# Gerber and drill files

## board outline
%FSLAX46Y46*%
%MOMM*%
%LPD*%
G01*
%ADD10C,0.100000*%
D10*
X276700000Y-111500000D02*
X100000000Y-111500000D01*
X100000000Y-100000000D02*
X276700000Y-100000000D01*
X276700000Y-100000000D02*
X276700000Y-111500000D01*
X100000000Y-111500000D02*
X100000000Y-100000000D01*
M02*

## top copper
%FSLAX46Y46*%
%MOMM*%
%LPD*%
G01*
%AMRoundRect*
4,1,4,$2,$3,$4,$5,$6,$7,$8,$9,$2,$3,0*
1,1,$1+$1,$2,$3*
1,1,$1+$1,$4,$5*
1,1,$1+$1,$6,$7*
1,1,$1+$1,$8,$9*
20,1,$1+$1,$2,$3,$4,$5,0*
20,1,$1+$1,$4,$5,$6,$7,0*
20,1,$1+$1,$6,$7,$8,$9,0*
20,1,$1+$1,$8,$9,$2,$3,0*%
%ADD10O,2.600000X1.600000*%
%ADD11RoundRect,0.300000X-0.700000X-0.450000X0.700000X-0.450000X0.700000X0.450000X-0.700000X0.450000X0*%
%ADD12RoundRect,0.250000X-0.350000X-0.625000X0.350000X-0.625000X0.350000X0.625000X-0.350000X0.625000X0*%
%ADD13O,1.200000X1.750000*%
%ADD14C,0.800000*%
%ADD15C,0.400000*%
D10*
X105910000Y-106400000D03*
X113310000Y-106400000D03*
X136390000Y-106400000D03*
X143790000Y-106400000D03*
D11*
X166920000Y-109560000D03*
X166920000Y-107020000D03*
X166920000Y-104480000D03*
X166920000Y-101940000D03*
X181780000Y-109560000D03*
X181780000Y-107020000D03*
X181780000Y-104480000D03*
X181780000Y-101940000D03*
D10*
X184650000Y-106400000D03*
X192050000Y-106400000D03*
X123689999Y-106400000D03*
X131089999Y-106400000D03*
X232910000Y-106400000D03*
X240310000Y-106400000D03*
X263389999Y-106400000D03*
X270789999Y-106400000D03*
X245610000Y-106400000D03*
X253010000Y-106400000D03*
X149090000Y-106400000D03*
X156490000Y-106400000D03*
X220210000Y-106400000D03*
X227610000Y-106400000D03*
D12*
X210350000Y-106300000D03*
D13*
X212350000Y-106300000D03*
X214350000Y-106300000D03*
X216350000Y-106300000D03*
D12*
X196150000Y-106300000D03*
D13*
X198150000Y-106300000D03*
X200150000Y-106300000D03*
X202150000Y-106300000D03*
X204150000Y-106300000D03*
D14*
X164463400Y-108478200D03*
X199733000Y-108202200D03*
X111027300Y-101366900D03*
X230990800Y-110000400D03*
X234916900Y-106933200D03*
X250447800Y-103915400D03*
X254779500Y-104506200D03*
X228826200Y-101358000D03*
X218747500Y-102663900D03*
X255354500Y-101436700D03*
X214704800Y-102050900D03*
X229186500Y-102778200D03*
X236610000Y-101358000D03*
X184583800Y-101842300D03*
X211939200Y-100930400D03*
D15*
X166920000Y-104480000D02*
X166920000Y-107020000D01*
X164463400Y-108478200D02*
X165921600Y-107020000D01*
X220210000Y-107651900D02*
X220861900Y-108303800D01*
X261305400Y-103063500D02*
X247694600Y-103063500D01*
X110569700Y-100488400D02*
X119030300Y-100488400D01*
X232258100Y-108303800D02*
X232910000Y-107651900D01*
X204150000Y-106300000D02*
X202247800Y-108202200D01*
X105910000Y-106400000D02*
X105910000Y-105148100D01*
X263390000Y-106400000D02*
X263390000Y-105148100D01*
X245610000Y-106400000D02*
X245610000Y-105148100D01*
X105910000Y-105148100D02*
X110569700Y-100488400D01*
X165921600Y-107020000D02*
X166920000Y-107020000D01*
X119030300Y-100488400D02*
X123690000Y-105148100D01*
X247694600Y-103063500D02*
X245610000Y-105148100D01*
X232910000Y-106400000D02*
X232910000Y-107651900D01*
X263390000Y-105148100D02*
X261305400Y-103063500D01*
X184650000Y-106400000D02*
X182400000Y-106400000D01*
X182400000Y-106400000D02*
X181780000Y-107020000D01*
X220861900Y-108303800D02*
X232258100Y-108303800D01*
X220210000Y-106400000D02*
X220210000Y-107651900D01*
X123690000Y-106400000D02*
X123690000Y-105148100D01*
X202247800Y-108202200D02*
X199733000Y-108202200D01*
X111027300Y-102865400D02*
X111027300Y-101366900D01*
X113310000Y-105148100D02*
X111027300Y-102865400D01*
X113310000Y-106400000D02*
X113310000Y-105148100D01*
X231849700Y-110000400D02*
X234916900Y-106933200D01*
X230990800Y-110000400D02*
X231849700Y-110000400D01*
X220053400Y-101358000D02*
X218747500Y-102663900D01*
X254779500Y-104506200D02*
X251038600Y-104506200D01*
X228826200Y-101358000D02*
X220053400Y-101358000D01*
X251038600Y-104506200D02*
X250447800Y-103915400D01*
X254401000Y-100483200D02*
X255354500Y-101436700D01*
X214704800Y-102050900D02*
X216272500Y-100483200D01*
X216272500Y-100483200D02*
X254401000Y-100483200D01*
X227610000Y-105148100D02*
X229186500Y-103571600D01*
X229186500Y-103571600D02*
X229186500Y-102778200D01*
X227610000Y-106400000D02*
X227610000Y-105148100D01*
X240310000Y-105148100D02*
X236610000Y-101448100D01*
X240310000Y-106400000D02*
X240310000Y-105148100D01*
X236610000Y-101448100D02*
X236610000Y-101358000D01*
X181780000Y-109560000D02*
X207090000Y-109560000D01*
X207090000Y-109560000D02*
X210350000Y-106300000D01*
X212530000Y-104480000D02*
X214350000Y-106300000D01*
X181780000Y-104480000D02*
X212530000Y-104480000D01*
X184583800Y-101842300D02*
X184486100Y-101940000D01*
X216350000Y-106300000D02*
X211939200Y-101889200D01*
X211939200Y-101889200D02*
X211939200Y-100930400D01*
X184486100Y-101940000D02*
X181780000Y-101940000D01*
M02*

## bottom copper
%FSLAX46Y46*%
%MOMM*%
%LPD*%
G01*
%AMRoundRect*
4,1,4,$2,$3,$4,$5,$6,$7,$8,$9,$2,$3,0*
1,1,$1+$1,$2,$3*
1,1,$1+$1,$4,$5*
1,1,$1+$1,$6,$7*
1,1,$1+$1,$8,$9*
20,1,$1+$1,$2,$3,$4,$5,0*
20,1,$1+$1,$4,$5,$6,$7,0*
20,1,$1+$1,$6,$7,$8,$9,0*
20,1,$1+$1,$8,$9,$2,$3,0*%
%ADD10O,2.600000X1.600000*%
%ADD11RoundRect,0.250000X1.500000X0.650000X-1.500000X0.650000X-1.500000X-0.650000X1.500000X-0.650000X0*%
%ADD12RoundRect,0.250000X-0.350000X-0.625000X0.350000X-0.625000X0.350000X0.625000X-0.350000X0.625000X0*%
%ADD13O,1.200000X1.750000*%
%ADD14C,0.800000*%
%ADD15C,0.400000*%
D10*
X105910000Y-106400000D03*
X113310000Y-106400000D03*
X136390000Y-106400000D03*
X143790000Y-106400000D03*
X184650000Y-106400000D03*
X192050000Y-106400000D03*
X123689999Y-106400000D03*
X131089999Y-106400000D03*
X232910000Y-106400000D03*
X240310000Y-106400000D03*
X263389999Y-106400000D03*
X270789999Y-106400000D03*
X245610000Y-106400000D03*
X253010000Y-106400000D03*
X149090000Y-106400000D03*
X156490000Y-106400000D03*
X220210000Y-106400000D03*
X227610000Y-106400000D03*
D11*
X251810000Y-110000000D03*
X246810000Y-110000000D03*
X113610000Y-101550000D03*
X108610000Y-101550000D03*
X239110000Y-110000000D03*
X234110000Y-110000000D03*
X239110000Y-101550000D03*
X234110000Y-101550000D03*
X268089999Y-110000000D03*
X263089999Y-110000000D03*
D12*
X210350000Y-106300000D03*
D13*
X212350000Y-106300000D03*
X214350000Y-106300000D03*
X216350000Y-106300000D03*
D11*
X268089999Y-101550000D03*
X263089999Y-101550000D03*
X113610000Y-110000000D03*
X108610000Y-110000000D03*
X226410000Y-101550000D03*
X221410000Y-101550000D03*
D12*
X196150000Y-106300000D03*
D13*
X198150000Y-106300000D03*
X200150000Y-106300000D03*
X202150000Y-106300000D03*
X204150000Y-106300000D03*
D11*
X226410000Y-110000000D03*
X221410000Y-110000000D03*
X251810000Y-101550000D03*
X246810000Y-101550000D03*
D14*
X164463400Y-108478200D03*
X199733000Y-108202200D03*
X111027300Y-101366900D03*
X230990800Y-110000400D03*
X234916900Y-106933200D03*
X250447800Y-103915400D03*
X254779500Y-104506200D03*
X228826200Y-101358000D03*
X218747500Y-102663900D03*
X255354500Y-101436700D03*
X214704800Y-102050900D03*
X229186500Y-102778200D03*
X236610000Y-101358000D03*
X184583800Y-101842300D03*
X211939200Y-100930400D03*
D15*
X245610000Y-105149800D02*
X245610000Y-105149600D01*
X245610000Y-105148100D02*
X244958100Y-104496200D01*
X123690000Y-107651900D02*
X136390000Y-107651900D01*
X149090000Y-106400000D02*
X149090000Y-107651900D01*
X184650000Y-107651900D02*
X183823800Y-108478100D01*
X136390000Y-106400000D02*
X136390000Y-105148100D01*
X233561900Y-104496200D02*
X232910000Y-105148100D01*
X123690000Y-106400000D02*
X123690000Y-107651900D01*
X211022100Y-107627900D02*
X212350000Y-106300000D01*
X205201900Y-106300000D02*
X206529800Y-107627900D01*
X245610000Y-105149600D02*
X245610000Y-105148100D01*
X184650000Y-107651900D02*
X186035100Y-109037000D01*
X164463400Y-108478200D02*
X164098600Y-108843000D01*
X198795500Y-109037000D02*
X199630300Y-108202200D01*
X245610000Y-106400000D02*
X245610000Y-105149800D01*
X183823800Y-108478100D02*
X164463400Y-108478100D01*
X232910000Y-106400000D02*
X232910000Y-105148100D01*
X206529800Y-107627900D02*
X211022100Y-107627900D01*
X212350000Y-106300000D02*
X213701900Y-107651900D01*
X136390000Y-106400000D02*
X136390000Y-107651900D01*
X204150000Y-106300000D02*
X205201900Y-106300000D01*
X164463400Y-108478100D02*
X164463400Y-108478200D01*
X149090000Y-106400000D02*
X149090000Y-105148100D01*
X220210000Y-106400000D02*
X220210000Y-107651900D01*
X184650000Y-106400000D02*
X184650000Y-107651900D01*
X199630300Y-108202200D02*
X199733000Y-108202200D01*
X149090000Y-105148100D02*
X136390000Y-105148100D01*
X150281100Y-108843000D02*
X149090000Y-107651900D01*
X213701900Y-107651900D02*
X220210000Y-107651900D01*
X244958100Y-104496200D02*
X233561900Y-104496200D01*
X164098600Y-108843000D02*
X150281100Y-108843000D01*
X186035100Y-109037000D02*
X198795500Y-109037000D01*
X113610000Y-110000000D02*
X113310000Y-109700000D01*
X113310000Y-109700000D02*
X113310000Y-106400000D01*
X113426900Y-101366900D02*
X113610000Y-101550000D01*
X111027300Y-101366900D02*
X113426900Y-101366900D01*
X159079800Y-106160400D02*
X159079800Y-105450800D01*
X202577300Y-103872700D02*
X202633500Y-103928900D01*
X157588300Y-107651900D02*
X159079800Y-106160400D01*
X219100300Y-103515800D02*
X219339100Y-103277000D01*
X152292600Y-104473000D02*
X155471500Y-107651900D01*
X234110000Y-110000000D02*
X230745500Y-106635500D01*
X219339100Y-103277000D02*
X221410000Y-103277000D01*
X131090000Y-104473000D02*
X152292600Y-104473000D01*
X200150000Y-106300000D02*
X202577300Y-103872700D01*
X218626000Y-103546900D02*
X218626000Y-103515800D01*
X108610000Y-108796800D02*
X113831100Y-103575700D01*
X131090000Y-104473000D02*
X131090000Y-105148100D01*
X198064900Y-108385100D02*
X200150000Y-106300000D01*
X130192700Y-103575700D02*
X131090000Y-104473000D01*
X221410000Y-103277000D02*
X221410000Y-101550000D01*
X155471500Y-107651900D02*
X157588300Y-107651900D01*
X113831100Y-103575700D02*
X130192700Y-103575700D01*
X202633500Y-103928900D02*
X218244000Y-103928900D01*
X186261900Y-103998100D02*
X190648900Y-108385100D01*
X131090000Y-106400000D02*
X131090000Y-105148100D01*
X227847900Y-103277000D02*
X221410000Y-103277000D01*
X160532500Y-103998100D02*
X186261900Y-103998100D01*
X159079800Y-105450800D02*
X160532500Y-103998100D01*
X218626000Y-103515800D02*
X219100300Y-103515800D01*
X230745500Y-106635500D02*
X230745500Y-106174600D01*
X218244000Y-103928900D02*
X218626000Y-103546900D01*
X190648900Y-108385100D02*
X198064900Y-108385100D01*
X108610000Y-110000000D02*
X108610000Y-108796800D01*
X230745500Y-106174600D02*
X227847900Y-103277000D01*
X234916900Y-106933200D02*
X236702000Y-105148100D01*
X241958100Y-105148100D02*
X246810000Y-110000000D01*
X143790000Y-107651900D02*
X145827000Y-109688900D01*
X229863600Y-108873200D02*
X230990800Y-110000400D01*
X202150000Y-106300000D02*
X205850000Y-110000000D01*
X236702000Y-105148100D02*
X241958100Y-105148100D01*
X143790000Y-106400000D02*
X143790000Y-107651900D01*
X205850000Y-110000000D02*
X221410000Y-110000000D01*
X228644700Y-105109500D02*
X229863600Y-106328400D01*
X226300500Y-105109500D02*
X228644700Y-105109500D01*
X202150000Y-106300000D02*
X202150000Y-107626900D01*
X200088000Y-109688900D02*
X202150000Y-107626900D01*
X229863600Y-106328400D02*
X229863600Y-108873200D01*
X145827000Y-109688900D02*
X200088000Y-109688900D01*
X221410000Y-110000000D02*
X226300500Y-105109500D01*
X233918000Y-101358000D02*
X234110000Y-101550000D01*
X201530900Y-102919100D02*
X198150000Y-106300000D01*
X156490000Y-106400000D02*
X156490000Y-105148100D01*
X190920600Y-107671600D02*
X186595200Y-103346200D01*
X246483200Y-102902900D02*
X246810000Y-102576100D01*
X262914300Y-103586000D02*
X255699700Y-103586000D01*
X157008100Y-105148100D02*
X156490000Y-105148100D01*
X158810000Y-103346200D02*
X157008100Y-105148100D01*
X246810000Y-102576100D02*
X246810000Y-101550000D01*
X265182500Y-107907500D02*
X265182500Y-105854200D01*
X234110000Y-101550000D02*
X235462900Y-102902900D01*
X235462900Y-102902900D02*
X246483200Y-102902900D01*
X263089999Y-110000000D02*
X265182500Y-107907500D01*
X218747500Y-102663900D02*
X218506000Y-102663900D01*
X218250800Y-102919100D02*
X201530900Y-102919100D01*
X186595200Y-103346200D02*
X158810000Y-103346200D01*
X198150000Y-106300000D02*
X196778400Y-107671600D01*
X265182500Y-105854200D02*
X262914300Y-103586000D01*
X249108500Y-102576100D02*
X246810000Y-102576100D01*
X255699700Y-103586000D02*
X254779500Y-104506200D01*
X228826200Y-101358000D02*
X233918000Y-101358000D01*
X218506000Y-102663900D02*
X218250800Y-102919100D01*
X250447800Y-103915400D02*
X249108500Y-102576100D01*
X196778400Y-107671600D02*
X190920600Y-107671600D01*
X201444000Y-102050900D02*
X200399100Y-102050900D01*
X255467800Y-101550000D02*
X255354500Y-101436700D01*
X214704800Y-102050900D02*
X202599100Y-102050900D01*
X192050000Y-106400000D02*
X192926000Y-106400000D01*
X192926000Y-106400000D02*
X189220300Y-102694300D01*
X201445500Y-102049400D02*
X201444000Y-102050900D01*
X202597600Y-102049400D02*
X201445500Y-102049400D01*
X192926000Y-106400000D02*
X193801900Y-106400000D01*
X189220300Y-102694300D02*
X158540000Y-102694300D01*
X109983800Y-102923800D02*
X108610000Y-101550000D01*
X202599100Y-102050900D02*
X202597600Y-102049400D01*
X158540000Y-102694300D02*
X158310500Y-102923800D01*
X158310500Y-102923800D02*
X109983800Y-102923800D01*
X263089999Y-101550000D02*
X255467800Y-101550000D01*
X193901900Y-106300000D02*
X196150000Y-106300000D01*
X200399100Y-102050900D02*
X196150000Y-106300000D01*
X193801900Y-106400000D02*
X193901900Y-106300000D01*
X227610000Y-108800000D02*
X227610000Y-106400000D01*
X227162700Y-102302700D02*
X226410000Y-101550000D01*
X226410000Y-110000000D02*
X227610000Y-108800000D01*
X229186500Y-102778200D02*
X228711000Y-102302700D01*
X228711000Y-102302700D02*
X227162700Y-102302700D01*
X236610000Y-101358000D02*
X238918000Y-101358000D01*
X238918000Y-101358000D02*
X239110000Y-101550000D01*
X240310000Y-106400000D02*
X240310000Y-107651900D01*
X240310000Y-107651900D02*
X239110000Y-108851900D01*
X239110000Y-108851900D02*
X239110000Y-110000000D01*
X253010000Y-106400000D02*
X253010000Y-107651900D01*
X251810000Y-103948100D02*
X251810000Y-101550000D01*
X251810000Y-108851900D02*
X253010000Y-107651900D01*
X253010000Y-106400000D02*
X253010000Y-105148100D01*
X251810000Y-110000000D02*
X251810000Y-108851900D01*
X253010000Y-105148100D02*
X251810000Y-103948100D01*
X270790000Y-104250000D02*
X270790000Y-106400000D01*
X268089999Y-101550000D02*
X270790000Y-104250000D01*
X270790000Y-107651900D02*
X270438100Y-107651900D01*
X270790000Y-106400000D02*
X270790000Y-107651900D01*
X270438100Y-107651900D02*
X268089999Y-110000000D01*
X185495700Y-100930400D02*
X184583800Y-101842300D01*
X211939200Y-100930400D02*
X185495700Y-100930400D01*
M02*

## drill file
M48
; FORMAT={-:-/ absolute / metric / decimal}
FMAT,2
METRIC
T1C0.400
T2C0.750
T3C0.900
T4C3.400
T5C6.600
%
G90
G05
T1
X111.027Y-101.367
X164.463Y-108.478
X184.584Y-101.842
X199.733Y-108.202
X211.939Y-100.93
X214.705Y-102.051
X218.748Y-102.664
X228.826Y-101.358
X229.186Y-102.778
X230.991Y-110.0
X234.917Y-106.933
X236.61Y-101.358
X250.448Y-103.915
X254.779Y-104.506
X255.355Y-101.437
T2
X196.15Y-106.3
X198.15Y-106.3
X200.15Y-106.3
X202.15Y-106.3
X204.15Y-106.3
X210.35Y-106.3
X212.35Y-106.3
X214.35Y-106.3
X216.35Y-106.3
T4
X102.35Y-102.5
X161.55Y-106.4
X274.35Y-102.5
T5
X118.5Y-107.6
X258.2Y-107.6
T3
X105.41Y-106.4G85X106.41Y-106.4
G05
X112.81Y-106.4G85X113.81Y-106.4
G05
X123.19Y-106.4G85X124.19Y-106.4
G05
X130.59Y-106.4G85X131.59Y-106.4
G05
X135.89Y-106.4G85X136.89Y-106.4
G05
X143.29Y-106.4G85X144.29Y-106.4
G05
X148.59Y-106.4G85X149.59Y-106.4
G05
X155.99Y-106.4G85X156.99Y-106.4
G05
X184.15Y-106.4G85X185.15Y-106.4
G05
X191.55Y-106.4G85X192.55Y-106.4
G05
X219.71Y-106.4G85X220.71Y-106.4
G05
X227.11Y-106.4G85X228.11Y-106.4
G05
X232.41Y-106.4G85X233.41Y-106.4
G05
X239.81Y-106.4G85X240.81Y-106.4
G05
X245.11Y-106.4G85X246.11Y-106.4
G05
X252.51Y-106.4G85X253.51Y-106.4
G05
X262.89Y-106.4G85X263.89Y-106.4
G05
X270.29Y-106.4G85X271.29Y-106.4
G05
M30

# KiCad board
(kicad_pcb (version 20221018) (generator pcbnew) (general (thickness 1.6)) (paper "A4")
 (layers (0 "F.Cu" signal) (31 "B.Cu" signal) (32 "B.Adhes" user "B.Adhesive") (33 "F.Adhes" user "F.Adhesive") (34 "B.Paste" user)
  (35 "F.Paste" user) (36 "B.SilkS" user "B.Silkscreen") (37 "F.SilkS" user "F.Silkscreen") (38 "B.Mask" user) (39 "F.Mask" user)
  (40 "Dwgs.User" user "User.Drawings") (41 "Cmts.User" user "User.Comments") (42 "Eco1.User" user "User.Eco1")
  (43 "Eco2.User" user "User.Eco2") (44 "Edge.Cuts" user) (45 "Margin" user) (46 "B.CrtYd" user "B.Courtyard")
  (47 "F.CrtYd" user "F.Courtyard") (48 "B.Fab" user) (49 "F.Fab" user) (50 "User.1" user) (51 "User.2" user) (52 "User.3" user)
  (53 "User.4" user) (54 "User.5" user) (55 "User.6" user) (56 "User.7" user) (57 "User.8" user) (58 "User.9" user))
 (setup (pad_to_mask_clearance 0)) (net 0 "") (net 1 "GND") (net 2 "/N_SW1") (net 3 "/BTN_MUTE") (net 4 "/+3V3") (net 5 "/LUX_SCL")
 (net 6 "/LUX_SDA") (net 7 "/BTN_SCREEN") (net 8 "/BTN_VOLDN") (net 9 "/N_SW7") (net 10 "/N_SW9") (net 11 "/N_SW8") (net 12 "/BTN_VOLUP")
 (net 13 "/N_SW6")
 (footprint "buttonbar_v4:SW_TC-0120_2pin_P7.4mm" (layer "F.Cu") (at 109.61 106.4)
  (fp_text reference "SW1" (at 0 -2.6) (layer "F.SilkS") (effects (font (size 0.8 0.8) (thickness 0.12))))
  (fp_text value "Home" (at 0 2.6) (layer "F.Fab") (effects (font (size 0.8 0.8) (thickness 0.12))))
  (pad "1" thru_hole oval (at -3.7 0) (size 2.6 1.6) (drill oval 1.9 0.9) (layers "*.Cu" "*.Mask") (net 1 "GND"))
  (pad "2" thru_hole oval (at 3.7 0) (size 2.6 1.6) (drill oval 1.9 0.9) (layers "*.Cu" "*.Mask") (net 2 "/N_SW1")))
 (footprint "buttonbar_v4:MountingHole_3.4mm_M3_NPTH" (layer "F.Cu") (at 274.35 102.5)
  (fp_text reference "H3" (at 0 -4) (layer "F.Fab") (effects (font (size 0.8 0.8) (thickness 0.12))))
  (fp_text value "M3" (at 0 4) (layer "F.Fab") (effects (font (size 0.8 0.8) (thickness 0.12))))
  (pad "" np_thru_hole circle (at 0 0) (size 3.4 3.4) (drill 3.4) (layers "*.Cu" "*.Mask")))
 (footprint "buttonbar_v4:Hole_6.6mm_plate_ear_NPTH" (layer "F.Cu") (at 118.5 107.6)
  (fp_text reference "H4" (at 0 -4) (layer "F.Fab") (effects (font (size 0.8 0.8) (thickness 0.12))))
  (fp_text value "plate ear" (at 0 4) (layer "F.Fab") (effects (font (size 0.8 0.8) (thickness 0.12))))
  (pad "" np_thru_hole circle (at 0 0) (size 6.6 6.6) (drill 6.6) (layers "*.Cu" "*.Mask")))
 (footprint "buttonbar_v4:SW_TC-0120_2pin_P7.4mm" (layer "F.Cu") (at 140.09 106.4)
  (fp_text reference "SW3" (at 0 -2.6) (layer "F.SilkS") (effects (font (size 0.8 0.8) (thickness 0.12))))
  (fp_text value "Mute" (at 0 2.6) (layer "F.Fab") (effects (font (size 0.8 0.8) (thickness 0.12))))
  (pad "1" thru_hole oval (at -3.7 0) (size 2.6 1.6) (drill oval 1.9 0.9) (layers "*.Cu" "*.Mask") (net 1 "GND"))
  (pad "2" thru_hole oval (at 3.7 0) (size 2.6 1.6) (drill oval 1.9 0.9) (layers "*.Cu" "*.Mask") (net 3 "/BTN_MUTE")))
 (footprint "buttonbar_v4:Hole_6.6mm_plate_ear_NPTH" (layer "F.Cu") (at 258.2 107.6)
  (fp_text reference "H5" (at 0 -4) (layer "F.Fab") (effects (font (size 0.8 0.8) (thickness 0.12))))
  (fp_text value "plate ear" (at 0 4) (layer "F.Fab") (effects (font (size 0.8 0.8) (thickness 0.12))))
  (pad "" np_thru_hole circle (at 0 0) (size 6.6 6.6) (drill 6.6) (layers "*.Cu" "*.Mask")))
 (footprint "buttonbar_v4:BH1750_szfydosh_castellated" (layer "F.Cu") (at 174.35 105.75) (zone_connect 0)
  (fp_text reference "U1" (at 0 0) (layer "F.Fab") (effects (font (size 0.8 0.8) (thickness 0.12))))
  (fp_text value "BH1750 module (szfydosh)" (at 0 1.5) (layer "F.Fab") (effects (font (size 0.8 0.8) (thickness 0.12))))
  (pad "1" smd roundrect (at -7.43 3.81) (size 2 1.5) (layers "F.Cu" "F.Paste" "F.Mask") (roundrect_rratio 0.2))
  (pad "2" smd roundrect (at -7.43 1.27) (size 2 1.5) (layers "F.Cu" "F.Paste" "F.Mask") (roundrect_rratio 0.2) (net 1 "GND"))
  (pad "3" smd roundrect (at -7.43 -1.27) (size 2 1.5) (layers "F.Cu" "F.Paste" "F.Mask") (roundrect_rratio 0.2) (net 1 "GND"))
  (pad "4" smd roundrect (at -7.43 -3.81) (size 2 1.5) (layers "F.Cu" "F.Paste" "F.Mask") (roundrect_rratio 0.2))
  (pad "5" smd roundrect (at 7.43 3.81) (size 2 1.5) (layers "F.Cu" "F.Paste" "F.Mask") (roundrect_rratio 0.2) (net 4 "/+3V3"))
  (pad "6" smd roundrect (at 7.43 1.27) (size 2 1.5) (layers "F.Cu" "F.Paste" "F.Mask") (roundrect_rratio 0.2) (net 1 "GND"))
  (pad "7" smd roundrect (at 7.43 -1.27) (size 2 1.5) (layers "F.Cu" "F.Paste" "F.Mask") (roundrect_rratio 0.2) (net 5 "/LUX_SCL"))
  (pad "8" smd roundrect (at 7.43 -3.81) (size 2 1.5) (layers "F.Cu" "F.Paste" "F.Mask") (roundrect_rratio 0.2) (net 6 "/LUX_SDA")))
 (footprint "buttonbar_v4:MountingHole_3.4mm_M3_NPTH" (layer "F.Cu") (at 102.35 102.5)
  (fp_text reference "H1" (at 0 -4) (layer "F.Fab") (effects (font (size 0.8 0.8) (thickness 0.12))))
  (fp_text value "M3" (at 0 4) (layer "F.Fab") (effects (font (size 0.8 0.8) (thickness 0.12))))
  (pad "" np_thru_hole circle (at 0 0) (size 3.4 3.4) (drill 3.4) (layers "*.Cu" "*.Mask")))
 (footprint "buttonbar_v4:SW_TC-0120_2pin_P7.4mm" (layer "F.Cu") (at 188.35 106.4)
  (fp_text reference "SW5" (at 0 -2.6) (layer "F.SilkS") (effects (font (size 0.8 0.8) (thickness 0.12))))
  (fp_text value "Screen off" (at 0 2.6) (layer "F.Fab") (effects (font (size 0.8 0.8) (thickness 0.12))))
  (pad "1" thru_hole oval (at -3.7 0) (size 2.6 1.6) (drill oval 1.9 0.9) (layers "*.Cu" "*.Mask") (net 1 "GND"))
  (pad "2" thru_hole oval (at 3.7 0) (size 2.6 1.6) (drill oval 1.9 0.9) (layers "*.Cu" "*.Mask") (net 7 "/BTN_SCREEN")))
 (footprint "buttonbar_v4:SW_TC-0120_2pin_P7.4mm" (layer "F.Cu") (at 127.389999 106.4)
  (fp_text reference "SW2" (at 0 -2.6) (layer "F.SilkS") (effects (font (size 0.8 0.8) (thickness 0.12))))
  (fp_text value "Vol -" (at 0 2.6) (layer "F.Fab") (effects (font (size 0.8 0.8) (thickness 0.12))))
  (pad "1" thru_hole oval (at -3.7 0) (size 2.6 1.6) (drill oval 1.9 0.9) (layers "*.Cu" "*.Mask") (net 1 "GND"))
  (pad "2" thru_hole oval (at 3.7 0) (size 2.6 1.6) (drill oval 1.9 0.9) (layers "*.Cu" "*.Mask") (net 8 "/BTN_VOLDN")))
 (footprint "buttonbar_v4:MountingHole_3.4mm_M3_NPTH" (layer "F.Cu") (at 161.549999 106.4)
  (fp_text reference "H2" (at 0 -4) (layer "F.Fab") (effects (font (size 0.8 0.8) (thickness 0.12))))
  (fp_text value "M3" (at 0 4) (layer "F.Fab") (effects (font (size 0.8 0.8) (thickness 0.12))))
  (pad "" np_thru_hole circle (at 0 0) (size 3.4 3.4) (drill 3.4) (layers "*.Cu" "*.Mask")))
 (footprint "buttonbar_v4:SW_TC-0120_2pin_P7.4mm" (layer "F.Cu") (at 236.61 106.4)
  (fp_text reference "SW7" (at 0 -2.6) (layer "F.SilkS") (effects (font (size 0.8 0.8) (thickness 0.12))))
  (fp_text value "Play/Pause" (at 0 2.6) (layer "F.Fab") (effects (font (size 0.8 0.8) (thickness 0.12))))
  (pad "1" thru_hole oval (at -3.7 0) (size 2.6 1.6) (drill oval 1.9 0.9) (layers "*.Cu" "*.Mask") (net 1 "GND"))
  (pad "2" thru_hole oval (at 3.7 0) (size 2.6 1.6) (drill oval 1.9 0.9) (layers "*.Cu" "*.Mask") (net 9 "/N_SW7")))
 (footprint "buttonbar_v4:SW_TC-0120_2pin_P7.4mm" (layer "F.Cu") (at 267.089999 106.4)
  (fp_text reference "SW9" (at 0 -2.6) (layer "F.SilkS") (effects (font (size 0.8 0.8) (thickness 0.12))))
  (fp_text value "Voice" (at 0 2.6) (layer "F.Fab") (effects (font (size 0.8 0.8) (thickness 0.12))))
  (pad "1" thru_hole oval (at -3.7 0) (size 2.6 1.6) (drill oval 1.9 0.9) (layers "*.Cu" "*.Mask") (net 1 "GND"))
  (pad "2" thru_hole oval (at 3.7 0) (size 2.6 1.6) (drill oval 1.9 0.9) (layers "*.Cu" "*.Mask") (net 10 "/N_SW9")))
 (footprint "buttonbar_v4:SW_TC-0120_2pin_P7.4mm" (layer "F.Cu") (at 249.31 106.4)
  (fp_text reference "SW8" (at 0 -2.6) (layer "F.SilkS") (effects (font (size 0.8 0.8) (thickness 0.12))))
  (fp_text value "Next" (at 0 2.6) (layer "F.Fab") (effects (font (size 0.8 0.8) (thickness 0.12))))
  (pad "1" thru_hole oval (at -3.7 0) (size 2.6 1.6) (drill oval 1.9 0.9) (layers "*.Cu" "*.Mask") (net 1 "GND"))
  (pad "2" thru_hole oval (at 3.7 0) (size 2.6 1.6) (drill oval 1.9 0.9) (layers "*.Cu" "*.Mask") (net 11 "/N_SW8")))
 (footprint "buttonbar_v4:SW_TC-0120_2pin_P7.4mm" (layer "F.Cu") (at 152.79 106.4)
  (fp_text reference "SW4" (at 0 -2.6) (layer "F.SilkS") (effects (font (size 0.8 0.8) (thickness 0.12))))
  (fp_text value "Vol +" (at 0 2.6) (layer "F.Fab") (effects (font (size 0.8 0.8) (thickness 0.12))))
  (pad "1" thru_hole oval (at -3.7 0) (size 2.6 1.6) (drill oval 1.9 0.9) (layers "*.Cu" "*.Mask") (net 1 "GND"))
  (pad "2" thru_hole oval (at 3.7 0) (size 2.6 1.6) (drill oval 1.9 0.9) (layers "*.Cu" "*.Mask") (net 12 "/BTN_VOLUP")))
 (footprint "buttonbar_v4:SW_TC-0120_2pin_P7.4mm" (layer "F.Cu") (at 223.91 106.4)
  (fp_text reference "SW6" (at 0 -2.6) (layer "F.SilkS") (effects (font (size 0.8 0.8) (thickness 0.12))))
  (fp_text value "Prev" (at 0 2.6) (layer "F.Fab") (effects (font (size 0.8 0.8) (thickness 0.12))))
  (pad "1" thru_hole oval (at -3.7 0) (size 2.6 1.6) (drill oval 1.9 0.9) (layers "*.Cu" "*.Mask") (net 1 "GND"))
  (pad "2" thru_hole oval (at 3.7 0) (size 2.6 1.6) (drill oval 1.9 0.9) (layers "*.Cu" "*.Mask") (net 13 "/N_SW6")))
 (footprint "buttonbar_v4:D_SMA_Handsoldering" (layer "B.Cu") (at 249.31 110 180)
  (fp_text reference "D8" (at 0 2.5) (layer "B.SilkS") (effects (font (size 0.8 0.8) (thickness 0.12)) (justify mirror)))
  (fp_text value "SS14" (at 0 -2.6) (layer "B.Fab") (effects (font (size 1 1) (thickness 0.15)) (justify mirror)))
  (pad "1" smd roundrect (at -2.5 0 180) (size 3.5 1.8) (layers "B.Cu" "B.Paste" "B.Mask") (roundrect_rratio 0.1388888889) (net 11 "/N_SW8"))
  (pad "2" smd roundrect (at 2.5 0 180) (size 3.5 1.8) (layers "B.Cu" "B.Paste" "B.Mask") (roundrect_rratio 0.1388888889)
   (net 3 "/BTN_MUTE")))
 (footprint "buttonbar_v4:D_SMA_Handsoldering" (layer "B.Cu") (at 111.11 101.55 180)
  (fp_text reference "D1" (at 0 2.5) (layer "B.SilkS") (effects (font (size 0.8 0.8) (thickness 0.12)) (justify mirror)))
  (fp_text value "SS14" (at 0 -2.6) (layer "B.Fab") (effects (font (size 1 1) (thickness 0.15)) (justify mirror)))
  (pad "1" smd roundrect (at -2.5 0 180) (size 3.5 1.8) (layers "B.Cu" "B.Paste" "B.Mask") (roundrect_rratio 0.1388888889) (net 2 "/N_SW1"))
  (pad "2" smd roundrect (at 2.5 0 180) (size 3.5 1.8) (layers "B.Cu" "B.Paste" "B.Mask") (roundrect_rratio 0.1388888889)
   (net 7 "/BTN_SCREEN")))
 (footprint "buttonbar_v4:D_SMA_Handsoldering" (layer "B.Cu") (at 236.61 110 180)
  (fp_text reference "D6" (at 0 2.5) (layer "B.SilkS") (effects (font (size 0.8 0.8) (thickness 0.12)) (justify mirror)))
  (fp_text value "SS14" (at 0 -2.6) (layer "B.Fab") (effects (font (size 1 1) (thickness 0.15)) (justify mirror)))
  (pad "1" smd roundrect (at -2.5 0 180) (size 3.5 1.8) (layers "B.Cu" "B.Paste" "B.Mask") (roundrect_rratio 0.1388888889) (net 9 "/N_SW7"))
  (pad "2" smd roundrect (at 2.5 0 180) (size 3.5 1.8) (layers "B.Cu" "B.Paste" "B.Mask") (roundrect_rratio 0.1388888889)
   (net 8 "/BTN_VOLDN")))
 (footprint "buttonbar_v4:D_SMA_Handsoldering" (layer "B.Cu") (at 236.61 101.55 180)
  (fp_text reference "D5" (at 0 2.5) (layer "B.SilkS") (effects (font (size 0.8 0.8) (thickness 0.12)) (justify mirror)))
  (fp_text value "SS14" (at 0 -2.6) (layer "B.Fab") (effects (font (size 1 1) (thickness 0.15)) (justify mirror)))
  (pad "1" smd roundrect (at -2.5 0 180) (size 3.5 1.8) (layers "B.Cu" "B.Paste" "B.Mask") (roundrect_rratio 0.1388888889) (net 9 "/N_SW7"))
  (pad "2" smd roundrect (at 2.5 0 180) (size 3.5 1.8) (layers "B.Cu" "B.Paste" "B.Mask") (roundrect_rratio 0.1388888889)
   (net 12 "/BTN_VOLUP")))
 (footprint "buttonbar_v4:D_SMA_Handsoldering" (layer "B.Cu") (at 265.589999 110 180)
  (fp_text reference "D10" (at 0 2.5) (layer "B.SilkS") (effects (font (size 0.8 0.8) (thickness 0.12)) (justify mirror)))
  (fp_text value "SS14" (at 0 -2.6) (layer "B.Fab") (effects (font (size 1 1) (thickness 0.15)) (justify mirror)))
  (pad "1" smd roundrect (at -2.5 0 180) (size 3.5 1.8) (layers "B.Cu" "B.Paste" "B.Mask") (roundrect_rratio 0.1388888889) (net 10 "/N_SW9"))
  (pad "2" smd roundrect (at 2.5 0 180) (size 3.5 1.8) (layers "B.Cu" "B.Paste" "B.Mask") (roundrect_rratio 0.1388888889)
   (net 12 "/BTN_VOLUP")))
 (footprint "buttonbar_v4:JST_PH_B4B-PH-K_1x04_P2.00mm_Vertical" (layer "B.Cu") (at 210.35 106.3)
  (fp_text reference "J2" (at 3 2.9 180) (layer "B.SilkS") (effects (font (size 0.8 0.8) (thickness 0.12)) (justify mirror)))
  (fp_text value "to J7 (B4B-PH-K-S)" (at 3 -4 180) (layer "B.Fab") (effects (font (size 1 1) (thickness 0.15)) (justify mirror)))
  (pad "1" thru_hole roundrect (at 0 0) (size 1.2 1.75) (drill 0.75) (layers "*.Cu" "*.Mask") (roundrect_rratio 0.208333) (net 4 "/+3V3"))
  (pad "2" thru_hole oval (at 2 0) (size 1.2 1.75) (drill 0.75) (layers "*.Cu" "*.Mask") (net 1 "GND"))
  (pad "3" thru_hole oval (at 4 0) (size 1.2 1.75) (drill 0.75) (layers "*.Cu" "*.Mask") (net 5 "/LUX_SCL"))
  (pad "4" thru_hole oval (at 6 0) (size 1.2 1.75) (drill 0.75) (layers "*.Cu" "*.Mask") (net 6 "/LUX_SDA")))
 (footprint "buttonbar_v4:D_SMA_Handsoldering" (layer "B.Cu") (at 265.589999 101.55 180)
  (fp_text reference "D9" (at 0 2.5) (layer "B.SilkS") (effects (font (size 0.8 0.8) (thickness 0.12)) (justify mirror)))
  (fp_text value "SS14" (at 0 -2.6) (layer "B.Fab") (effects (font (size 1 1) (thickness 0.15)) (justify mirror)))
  (pad "1" smd roundrect (at -2.5 0 180) (size 3.5 1.8) (layers "B.Cu" "B.Paste" "B.Mask") (roundrect_rratio 0.1388888889) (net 10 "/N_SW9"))
  (pad "2" smd roundrect (at 2.5 0 180) (size 3.5 1.8) (layers "B.Cu" "B.Paste" "B.Mask") (roundrect_rratio 0.1388888889)
   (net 7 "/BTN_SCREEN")))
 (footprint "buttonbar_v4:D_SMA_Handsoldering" (layer "B.Cu") (at 111.11 110 180)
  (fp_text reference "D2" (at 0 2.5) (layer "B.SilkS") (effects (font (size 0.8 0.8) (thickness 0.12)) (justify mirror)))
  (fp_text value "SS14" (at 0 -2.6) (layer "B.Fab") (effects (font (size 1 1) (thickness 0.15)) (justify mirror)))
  (pad "1" smd roundrect (at -2.5 0 180) (size 3.5 1.8) (layers "B.Cu" "B.Paste" "B.Mask") (roundrect_rratio 0.1388888889) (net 2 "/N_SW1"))
  (pad "2" smd roundrect (at 2.5 0 180) (size 3.5 1.8) (layers "B.Cu" "B.Paste" "B.Mask") (roundrect_rratio 0.1388888889)
   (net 8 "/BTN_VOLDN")))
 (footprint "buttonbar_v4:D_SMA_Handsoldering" (layer "B.Cu") (at 223.91 101.55 180)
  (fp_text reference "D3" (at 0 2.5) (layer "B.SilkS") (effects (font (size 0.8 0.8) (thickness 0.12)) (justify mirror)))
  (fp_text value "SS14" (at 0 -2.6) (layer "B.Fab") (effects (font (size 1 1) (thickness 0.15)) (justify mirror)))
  (pad "1" smd roundrect (at -2.5 0 180) (size 3.5 1.8) (layers "B.Cu" "B.Paste" "B.Mask") (roundrect_rratio 0.1388888889) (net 13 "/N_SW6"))
  (pad "2" smd roundrect (at 2.5 0 180) (size 3.5 1.8) (layers "B.Cu" "B.Paste" "B.Mask") (roundrect_rratio 0.1388888889)
   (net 8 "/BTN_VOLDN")))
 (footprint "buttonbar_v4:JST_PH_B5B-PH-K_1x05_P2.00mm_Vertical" (layer "B.Cu") (at 196.15 106.3)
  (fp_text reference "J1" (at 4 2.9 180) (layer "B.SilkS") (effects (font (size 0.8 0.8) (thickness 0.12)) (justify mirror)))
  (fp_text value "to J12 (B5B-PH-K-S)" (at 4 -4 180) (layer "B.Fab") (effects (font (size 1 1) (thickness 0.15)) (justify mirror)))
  (pad "1" thru_hole roundrect (at 0 0) (size 1.2 1.75) (drill 0.75) (layers "*.Cu" "*.Mask") (roundrect_rratio 0.208333)
   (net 7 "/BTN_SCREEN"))
  (pad "2" thru_hole oval (at 2 0) (size 1.2 1.75) (drill 0.75) (layers "*.Cu" "*.Mask") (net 12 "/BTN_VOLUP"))
  (pad "3" thru_hole oval (at 4 0) (size 1.2 1.75) (drill 0.75) (layers "*.Cu" "*.Mask") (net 8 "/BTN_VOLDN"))
  (pad "4" thru_hole oval (at 6 0) (size 1.2 1.75) (drill 0.75) (layers "*.Cu" "*.Mask") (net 3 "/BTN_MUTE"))
  (pad "5" thru_hole oval (at 8 0) (size 1.2 1.75) (drill 0.75) (layers "*.Cu" "*.Mask") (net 1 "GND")))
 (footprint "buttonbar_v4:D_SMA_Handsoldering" (layer "B.Cu") (at 223.91 110 180)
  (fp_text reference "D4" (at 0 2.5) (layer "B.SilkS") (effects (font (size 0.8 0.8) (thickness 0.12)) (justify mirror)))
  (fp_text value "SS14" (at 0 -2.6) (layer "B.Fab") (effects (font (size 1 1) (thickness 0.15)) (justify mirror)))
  (pad "1" smd roundrect (at -2.5 0 180) (size 3.5 1.8) (layers "B.Cu" "B.Paste" "B.Mask") (roundrect_rratio 0.1388888889) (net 13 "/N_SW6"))
  (pad "2" smd roundrect (at 2.5 0 180) (size 3.5 1.8) (layers "B.Cu" "B.Paste" "B.Mask") (roundrect_rratio 0.1388888889)
   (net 3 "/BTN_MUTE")))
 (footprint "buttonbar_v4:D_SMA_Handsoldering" (layer "B.Cu") (at 249.31 101.55 180)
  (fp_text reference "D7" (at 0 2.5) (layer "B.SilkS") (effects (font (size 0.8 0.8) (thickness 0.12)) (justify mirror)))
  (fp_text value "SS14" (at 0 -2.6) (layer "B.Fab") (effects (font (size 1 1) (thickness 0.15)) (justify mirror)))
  (pad "1" smd roundrect (at -2.5 0 180) (size 3.5 1.8) (layers "B.Cu" "B.Paste" "B.Mask") (roundrect_rratio 0.1388888889) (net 11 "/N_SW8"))
  (pad "2" smd roundrect (at 2.5 0 180) (size 3.5 1.8) (layers "B.Cu" "B.Paste" "B.Mask") (roundrect_rratio 0.1388888889)
   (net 12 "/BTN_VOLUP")))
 (gr_line (start 276.7 111.5) (end 100 111.5) (stroke (width 0.1) (type default)) (layer "Edge.Cuts"))
 (gr_line (start 100 100) (end 276.7 100) (stroke (width 0.1) (type default)) (layer "Edge.Cuts"))
 (gr_line (start 276.7 100) (end 276.7 111.5) (stroke (width 0.1) (type default)) (layer "Edge.Cuts"))
 (gr_line (start 100 111.5) (end 100 100) (stroke (width 0.1) (type default)) (layer "Edge.Cuts"))
 (segment (start 166.92 104.48) (end 166.92 107.02) (width 0.4) (layer "F.Cu") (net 1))
 (segment (start 164.4634 108.4782) (end 165.9216 107.02) (width 0.4) (layer "F.Cu") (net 1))
 (segment (start 220.21 107.6519) (end 220.8619 108.3038) (width 0.4) (layer "F.Cu") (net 1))
 (segment (start 261.3054 103.0635) (end 247.6946 103.0635) (width 0.4) (layer "F.Cu") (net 1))
 (segment (start 110.5697 100.4884) (end 119.0303 100.4884) (width 0.4) (layer "F.Cu") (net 1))
 (segment (start 232.2581 108.3038) (end 232.91 107.6519) (width 0.4) (layer "F.Cu") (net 1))
 (segment (start 204.15 106.3) (end 202.2478 108.2022) (width 0.4) (layer "F.Cu") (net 1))
 (segment (start 105.91 106.4) (end 105.91 105.1481) (width 0.4) (layer "F.Cu") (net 1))
 (segment (start 263.39 106.4) (end 263.39 105.1481) (width 0.4) (layer "F.Cu") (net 1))
 (segment (start 245.61 106.4) (end 245.61 105.1481) (width 0.4) (layer "F.Cu") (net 1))
 (segment (start 105.91 105.1481) (end 110.5697 100.4884) (width 0.4) (layer "F.Cu") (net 1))
 (segment (start 165.9216 107.02) (end 166.92 107.02) (width 0.4) (layer "F.Cu") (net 1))
 (segment (start 119.0303 100.4884) (end 123.69 105.1481) (width 0.4) (layer "F.Cu") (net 1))
 (segment (start 247.6946 103.0635) (end 245.61 105.1481) (width 0.4) (layer "F.Cu") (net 1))
 (segment (start 232.91 106.4) (end 232.91 107.6519) (width 0.4) (layer "F.Cu") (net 1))
 (segment (start 263.39 105.1481) (end 261.3054 103.0635) (width 0.4) (layer "F.Cu") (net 1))
 (segment (start 184.65 106.4) (end 182.4 106.4) (width 0.4) (layer "F.Cu") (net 1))
 (segment (start 182.4 106.4) (end 181.78 107.02) (width 0.4) (layer "F.Cu") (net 1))
 (segment (start 220.8619 108.3038) (end 232.2581 108.3038) (width 0.4) (layer "F.Cu") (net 1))
 (segment (start 220.21 106.4) (end 220.21 107.6519) (width 0.4) (layer "F.Cu") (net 1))
 (segment (start 123.69 106.4) (end 123.69 105.1481) (width 0.4) (layer "F.Cu") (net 1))
 (segment (start 202.2478 108.2022) (end 199.733 108.2022) (width 0.4) (layer "F.Cu") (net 1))
 (via (at 164.4634 108.4782) (size 0.8) (drill 0.4) (layers "F.Cu" "B.Cu") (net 1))
 (via (at 199.733 108.2022) (size 0.8) (drill 0.4) (layers "F.Cu" "B.Cu") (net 1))
 (segment (start 245.61 105.1498) (end 245.61 105.1496) (width 0.4) (layer "B.Cu") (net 1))
 (segment (start 245.61 105.1481) (end 244.9581 104.4962) (width 0.4) (layer "B.Cu") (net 1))
 (segment (start 123.69 107.6519) (end 136.39 107.6519) (width 0.4) (layer "B.Cu") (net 1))
 (segment (start 149.09 106.4) (end 149.09 107.6519) (width 0.4) (layer "B.Cu") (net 1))
 (segment (start 184.65 107.6519) (end 183.8238 108.4781) (width 0.4) (layer "B.Cu") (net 1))
 (segment (start 136.39 106.4) (end 136.39 105.1481) (width 0.4) (layer "B.Cu") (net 1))
 (segment (start 233.5619 104.4962) (end 232.91 105.1481) (width 0.4) (layer "B.Cu") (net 1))
 (segment (start 123.69 106.4) (end 123.69 107.6519) (width 0.4) (layer "B.Cu") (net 1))
 (segment (start 211.0221 107.6279) (end 212.35 106.3) (width 0.4) (layer "B.Cu") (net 1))
 (segment (start 205.2019 106.3) (end 206.5298 107.6279) (width 0.4) (layer "B.Cu") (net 1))
 (segment (start 245.61 105.1496) (end 245.61 105.1481) (width 0.4) (layer "B.Cu") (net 1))
 (segment (start 184.65 107.6519) (end 186.0351 109.037) (width 0.4) (layer "B.Cu") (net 1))
 (segment (start 164.4634 108.4782) (end 164.0986 108.843) (width 0.4) (layer "B.Cu") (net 1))
 (segment (start 198.7955 109.037) (end 199.6303 108.2022) (width 0.4) (layer "B.Cu") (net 1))
 (segment (start 245.61 106.4) (end 245.61 105.1498) (width 0.4) (layer "B.Cu") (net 1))
 (segment (start 183.8238 108.4781) (end 164.4634 108.4781) (width 0.4) (layer "B.Cu") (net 1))
 (segment (start 232.91 106.4) (end 232.91 105.1481) (width 0.4) (layer "B.Cu") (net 1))
 (segment (start 206.5298 107.6279) (end 211.0221 107.6279) (width 0.4) (layer "B.Cu") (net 1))
 (segment (start 212.35 106.3) (end 213.7019 107.6519) (width 0.4) (layer "B.Cu") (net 1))
 (segment (start 136.39 106.4) (end 136.39 107.6519) (width 0.4) (layer "B.Cu") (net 1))
 (segment (start 204.15 106.3) (end 205.2019 106.3) (width 0.4) (layer "B.Cu") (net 1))
 (segment (start 164.4634 108.4781) (end 164.4634 108.4782) (width 0.4) (layer "B.Cu") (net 1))
 (segment (start 149.09 106.4) (end 149.09 105.1481) (width 0.4) (layer "B.Cu") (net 1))
 (segment (start 220.21 106.4) (end 220.21 107.6519) (width 0.4) (layer "B.Cu") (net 1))
 (segment (start 184.65 106.4) (end 184.65 107.6519) (width 0.4) (layer "B.Cu") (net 1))
 (segment (start 199.6303 108.2022) (end 199.733 108.2022) (width 0.4) (layer "B.Cu") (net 1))
 (segment (start 149.09 105.1481) (end 136.39 105.1481) (width 0.4) (layer "B.Cu") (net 1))
 (segment (start 150.2811 108.843) (end 149.09 107.6519) (width 0.4) (layer "B.Cu") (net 1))
 (segment (start 213.7019 107.6519) (end 220.21 107.6519) (width 0.4) (layer "B.Cu") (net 1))
 (segment (start 244.9581 104.4962) (end 233.5619 104.4962) (width 0.4) (layer "B.Cu") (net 1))
 (segment (start 164.0986 108.843) (end 150.2811 108.843) (width 0.4) (layer "B.Cu") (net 1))
 (segment (start 186.0351 109.037) (end 198.7955 109.037) (width 0.4) (layer "B.Cu") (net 1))
 (segment (start 111.0273 102.8654) (end 111.0273 101.3669) (width 0.4) (layer "F.Cu") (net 2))
 (segment (start 113.31 105.1481) (end 111.0273 102.8654) (width 0.4) (layer "F.Cu") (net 2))
 (segment (start 113.31 106.4) (end 113.31 105.1481) (width 0.4) (layer "F.Cu") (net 2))
 (via (at 111.0273 101.3669) (size 0.8) (drill 0.4) (layers "F.Cu" "B.Cu") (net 2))
 (segment (start 113.61 110) (end 113.31 109.7) (width 0.4) (layer "B.Cu") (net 2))
 (segment (start 113.31 109.7) (end 113.31 106.4) (width 0.4) (layer "B.Cu") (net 2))
 (segment (start 113.4269 101.3669) (end 113.61 101.55) (width 0.4) (layer "B.Cu") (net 2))
 (segment (start 111.0273 101.3669) (end 113.4269 101.3669) (width 0.4) (layer "B.Cu") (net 2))
 (segment (start 159.0798 106.1604) (end 159.0798 105.4508) (width 0.4) (layer "B.Cu") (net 8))
 (segment (start 202.5773 103.8727) (end 202.6335 103.9289) (width 0.4) (layer "B.Cu") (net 8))
 (segment (start 157.5883 107.6519) (end 159.0798 106.1604) (width 0.4) (layer "B.Cu") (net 8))
 (segment (start 219.1003 103.5158) (end 219.3391 103.277) (width 0.4) (layer "B.Cu") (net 8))
 (segment (start 152.2926 104.473) (end 155.4715 107.6519) (width 0.4) (layer "B.Cu") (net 8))
 (segment (start 234.11 110) (end 230.7455 106.6355) (width 0.4) (layer "B.Cu") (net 8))
 (segment (start 219.3391 103.277) (end 221.41 103.277) (width 0.4) (layer "B.Cu") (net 8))
 (segment (start 131.09 104.473) (end 152.2926 104.473) (width 0.4) (layer "B.Cu") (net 8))
 (segment (start 200.15 106.3) (end 202.5773 103.8727) (width 0.4) (layer "B.Cu") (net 8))
 (segment (start 218.626 103.5469) (end 218.626 103.5158) (width 0.4) (layer "B.Cu") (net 8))
 (segment (start 108.61 108.7968) (end 113.8311 103.5757) (width 0.4) (layer "B.Cu") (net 8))
 (segment (start 131.09 104.473) (end 131.09 105.1481) (width 0.4) (layer "B.Cu") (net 8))
 (segment (start 198.0649 108.3851) (end 200.15 106.3) (width 0.4) (layer "B.Cu") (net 8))
 (segment (start 130.1927 103.5757) (end 131.09 104.473) (width 0.4) (layer "B.Cu") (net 8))
 (segment (start 221.41 103.277) (end 221.41 101.55) (width 0.4) (layer "B.Cu") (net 8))
 (segment (start 155.4715 107.6519) (end 157.5883 107.6519) (width 0.4) (layer "B.Cu") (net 8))
 (segment (start 113.8311 103.5757) (end 130.1927 103.5757) (width 0.4) (layer "B.Cu") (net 8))
 (segment (start 202.6335 103.9289) (end 218.244 103.9289) (width 0.4) (layer "B.Cu") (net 8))
 (segment (start 186.2619 103.9981) (end 190.6489 108.3851) (width 0.4) (layer "B.Cu") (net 8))
 (segment (start 131.09 106.4) (end 131.09 105.1481) (width 0.4) (layer "B.Cu") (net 8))
 (segment (start 227.8479 103.277) (end 221.41 103.277) (width 0.4) (layer "B.Cu") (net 8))
 (segment (start 160.5325 103.9981) (end 186.2619 103.9981) (width 0.4) (layer "B.Cu") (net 8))
 (segment (start 159.0798 105.4508) (end 160.5325 103.9981) (width 0.4) (layer "B.Cu") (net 8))
 (segment (start 218.626 103.5158) (end 219.1003 103.5158) (width 0.4) (layer "B.Cu") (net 8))
 (segment (start 230.7455 106.6355) (end 230.7455 106.1746) (width 0.4) (layer "B.Cu") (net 8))
 (segment (start 218.244 103.9289) (end 218.626 103.5469) (width 0.4) (layer "B.Cu") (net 8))
 (segment (start 190.6489 108.3851) (end 198.0649 108.3851) (width 0.4) (layer "B.Cu") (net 8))
 (segment (start 108.61 110) (end 108.61 108.7968) (width 0.4) (layer "B.Cu") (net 8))
 (segment (start 230.7455 106.1746) (end 227.8479 103.277) (width 0.4) (layer "B.Cu") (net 8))
 (segment (start 231.8497 110.0004) (end 234.9169 106.9332) (width 0.4) (layer "F.Cu") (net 3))
 (segment (start 230.9908 110.0004) (end 231.8497 110.0004) (width 0.4) (layer "F.Cu") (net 3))
 (via (at 230.9908 110.0004) (size 0.8) (drill 0.4) (layers "F.Cu" "B.Cu") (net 3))
 (via (at 234.9169 106.9332) (size 0.8) (drill 0.4) (layers "F.Cu" "B.Cu") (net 3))
 (segment (start 234.9169 106.9332) (end 236.702 105.1481) (width 0.4) (layer "B.Cu") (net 3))
 (segment (start 241.9581 105.1481) (end 246.81 110) (width 0.4) (layer "B.Cu") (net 3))
 (segment (start 143.79 107.6519) (end 145.827 109.6889) (width 0.4) (layer "B.Cu") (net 3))
 (segment (start 229.8636 108.8732) (end 230.9908 110.0004) (width 0.4) (layer "B.Cu") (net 3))
 (segment (start 202.15 106.3) (end 205.85 110) (width 0.4) (layer "B.Cu") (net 3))
 (segment (start 236.702 105.1481) (end 241.9581 105.1481) (width 0.4) (layer "B.Cu") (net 3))
 (segment (start 143.79 106.4) (end 143.79 107.6519) (width 0.4) (layer "B.Cu") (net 3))
 (segment (start 205.85 110) (end 221.41 110) (width 0.4) (layer "B.Cu") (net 3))
 (segment (start 228.6447 105.1095) (end 229.8636 106.3284) (width 0.4) (layer "B.Cu") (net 3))
 (segment (start 226.3005 105.1095) (end 228.6447 105.1095) (width 0.4) (layer "B.Cu") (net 3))
 (segment (start 202.15 106.3) (end 202.15 107.6269) (width 0.4) (layer "B.Cu") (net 3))
 (segment (start 200.088 109.6889) (end 202.15 107.6269) (width 0.4) (layer "B.Cu") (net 3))
 (segment (start 229.8636 106.3284) (end 229.8636 108.8732) (width 0.4) (layer "B.Cu") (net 3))
 (segment (start 145.827 109.6889) (end 200.088 109.6889) (width 0.4) (layer "B.Cu") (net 3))
 (segment (start 221.41 110) (end 226.3005 105.1095) (width 0.4) (layer "B.Cu") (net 3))
 (segment (start 220.0534 101.358) (end 218.7475 102.6639) (width 0.4) (layer "F.Cu") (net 12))
 (segment (start 254.7795 104.5062) (end 251.0386 104.5062) (width 0.4) (layer "F.Cu") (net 12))
 (segment (start 228.8262 101.358) (end 220.0534 101.358) (width 0.4) (layer "F.Cu") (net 12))
 (segment (start 251.0386 104.5062) (end 250.4478 103.9154) (width 0.4) (layer "F.Cu") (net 12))
 (via (at 250.4478 103.9154) (size 0.8) (drill 0.4) (layers "F.Cu" "B.Cu") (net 12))
 (via (at 254.7795 104.5062) (size 0.8) (drill 0.4) (layers "F.Cu" "B.Cu") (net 12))
 (via (at 228.8262 101.358) (size 0.8) (drill 0.4) (layers "F.Cu" "B.Cu") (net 12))
 (via (at 218.7475 102.6639) (size 0.8) (drill 0.4) (layers "F.Cu" "B.Cu") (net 12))
 (segment (start 233.918 101.358) (end 234.11 101.55) (width 0.4) (layer "B.Cu") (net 12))
 (segment (start 201.5309 102.9191) (end 198.15 106.3) (width 0.4) (layer "B.Cu") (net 12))
 (segment (start 156.49 106.4) (end 156.49 105.1481) (width 0.4) (layer "B.Cu") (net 12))
 (segment (start 190.9206 107.6716) (end 186.5952 103.3462) (width 0.4) (layer "B.Cu") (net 12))
 (segment (start 246.4832 102.9029) (end 246.81 102.5761) (width 0.4) (layer "B.Cu") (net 12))
 (segment (start 262.9143 103.586) (end 255.6997 103.586) (width 0.4) (layer "B.Cu") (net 12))
 (segment (start 157.0081 105.1481) (end 156.49 105.1481) (width 0.4) (layer "B.Cu") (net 12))
 (segment (start 158.81 103.3462) (end 157.0081 105.1481) (width 0.4) (layer "B.Cu") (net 12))
 (segment (start 246.81 102.5761) (end 246.81 101.55) (width 0.4) (layer "B.Cu") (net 12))
 (segment (start 265.1825 107.9075) (end 265.1825 105.8542) (width 0.4) (layer "B.Cu") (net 12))
 (segment (start 234.11 101.55) (end 235.4629 102.9029) (width 0.4) (layer "B.Cu") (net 12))
 (segment (start 235.4629 102.9029) (end 246.4832 102.9029) (width 0.4) (layer "B.Cu") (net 12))
 (segment (start 263.089999 110) (end 265.1825 107.9075) (width 0.4) (layer "B.Cu") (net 12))
 (segment (start 218.7475 102.6639) (end 218.506 102.6639) (width 0.4) (layer "B.Cu") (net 12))
 (segment (start 218.2508 102.9191) (end 201.5309 102.9191) (width 0.4) (layer "B.Cu") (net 12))
 (segment (start 186.5952 103.3462) (end 158.81 103.3462) (width 0.4) (layer "B.Cu") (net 12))
 (segment (start 198.15 106.3) (end 196.7784 107.6716) (width 0.4) (layer "B.Cu") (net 12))
 (segment (start 265.1825 105.8542) (end 262.9143 103.586) (width 0.4) (layer "B.Cu") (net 12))
 (segment (start 249.1085 102.5761) (end 246.81 102.5761) (width 0.4) (layer "B.Cu") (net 12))
 (segment (start 255.6997 103.586) (end 254.7795 104.5062) (width 0.4) (layer "B.Cu") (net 12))
 (segment (start 228.8262 101.358) (end 233.918 101.358) (width 0.4) (layer "B.Cu") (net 12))
 (segment (start 218.506 102.6639) (end 218.2508 102.9191) (width 0.4) (layer "B.Cu") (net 12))
 (segment (start 250.4478 103.9154) (end 249.1085 102.5761) (width 0.4) (layer "B.Cu") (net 12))
 (segment (start 196.7784 107.6716) (end 190.9206 107.6716) (width 0.4) (layer "B.Cu") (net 12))
 (segment (start 254.401 100.4832) (end 255.3545 101.4367) (width 0.4) (layer "F.Cu") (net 7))
 (segment (start 214.7048 102.0509) (end 216.2725 100.4832) (width 0.4) (layer "F.Cu") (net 7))
 (segment (start 216.2725 100.4832) (end 254.401 100.4832) (width 0.4) (layer "F.Cu") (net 7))
 (via (at 255.3545 101.4367) (size 0.8) (drill 0.4) (layers "F.Cu" "B.Cu") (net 7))
 (via (at 214.7048 102.0509) (size 0.8) (drill 0.4) (layers "F.Cu" "B.Cu") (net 7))
 (segment (start 201.444 102.0509) (end 200.3991 102.0509) (width 0.4) (layer "B.Cu") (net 7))
 (segment (start 255.4678 101.55) (end 255.3545 101.4367) (width 0.4) (layer "B.Cu") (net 7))
 (segment (start 214.7048 102.0509) (end 202.5991 102.0509) (width 0.4) (layer "B.Cu") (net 7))
 (segment (start 192.05 106.4) (end 192.926 106.4) (width 0.4) (layer "B.Cu") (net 7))
 (segment (start 192.926 106.4) (end 189.2203 102.6943) (width 0.4) (layer "B.Cu") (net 7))
 (segment (start 201.4455 102.0494) (end 201.444 102.0509) (width 0.4) (layer "B.Cu") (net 7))
 (segment (start 202.5976 102.0494) (end 201.4455 102.0494) (width 0.4) (layer "B.Cu") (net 7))
 (segment (start 192.926 106.4) (end 193.8019 106.4) (width 0.4) (layer "B.Cu") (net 7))
 (segment (start 189.2203 102.6943) (end 158.54 102.6943) (width 0.4) (layer "B.Cu") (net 7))
 (segment (start 109.9838 102.9238) (end 108.61 101.55) (width 0.4) (layer "B.Cu") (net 7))
 (segment (start 202.5991 102.0509) (end 202.5976 102.0494) (width 0.4) (layer "B.Cu") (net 7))
 (segment (start 158.54 102.6943) (end 158.3105 102.9238) (width 0.4) (layer "B.Cu") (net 7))
 (segment (start 158.3105 102.9238) (end 109.9838 102.9238) (width 0.4) (layer "B.Cu") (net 7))
 (segment (start 263.089999 101.55) (end 255.4678 101.55) (width 0.4) (layer "B.Cu") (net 7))
 (segment (start 193.9019 106.3) (end 196.15 106.3) (width 0.4) (layer "B.Cu") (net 7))
 (segment (start 200.3991 102.0509) (end 196.15 106.3) (width 0.4) (layer "B.Cu") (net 7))
 (segment (start 193.8019 106.4) (end 193.9019 106.3) (width 0.4) (layer "B.Cu") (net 7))
 (segment (start 227.61 105.1481) (end 229.1865 103.5716) (width 0.4) (layer "F.Cu") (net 13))
 (segment (start 229.1865 103.5716) (end 229.1865 102.7782) (width 0.4) (layer "F.Cu") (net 13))
 (segment (start 227.61 106.4) (end 227.61 105.1481) (width 0.4) (layer "F.Cu") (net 13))
 (via (at 229.1865 102.7782) (size 0.8) (drill 0.4) (layers "F.Cu" "B.Cu") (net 13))
 (segment (start 227.61 108.8) (end 227.61 106.4) (width 0.4) (layer "B.Cu") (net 13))
 (segment (start 227.1627 102.3027) (end 226.41 101.55) (width 0.4) (layer "B.Cu") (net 13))
 (segment (start 226.41 110) (end 227.61 108.8) (width 0.4) (layer "B.Cu") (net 13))
 (segment (start 229.1865 102.7782) (end 228.711 102.3027) (width 0.4) (layer "B.Cu") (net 13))
 (segment (start 228.711 102.3027) (end 227.1627 102.3027) (width 0.4) (layer "B.Cu") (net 13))
 (segment (start 240.31 105.1481) (end 236.61 101.4481) (width 0.4) (layer "F.Cu") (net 9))
 (segment (start 240.31 106.4) (end 240.31 105.1481) (width 0.4) (layer "F.Cu") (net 9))
 (segment (start 236.61 101.4481) (end 236.61 101.358) (width 0.4) (layer "F.Cu") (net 9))
 (via (at 236.61 101.358) (size 0.8) (drill 0.4) (layers "F.Cu" "B.Cu") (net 9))
 (segment (start 236.61 101.358) (end 238.918 101.358) (width 0.4) (layer "B.Cu") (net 9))
 (segment (start 238.918 101.358) (end 239.11 101.55) (width 0.4) (layer "B.Cu") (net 9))
 (segment (start 240.31 106.4) (end 240.31 107.6519) (width 0.4) (layer "B.Cu") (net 9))
 (segment (start 240.31 107.6519) (end 239.11 108.8519) (width 0.4) (layer "B.Cu") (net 9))
 (segment (start 239.11 108.8519) (end 239.11 110) (width 0.4) (layer "B.Cu") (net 9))
 (segment (start 253.01 106.4) (end 253.01 107.6519) (width 0.4) (layer "B.Cu") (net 11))
 (segment (start 251.81 103.9481) (end 251.81 101.55) (width 0.4) (layer "B.Cu") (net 11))
 (segment (start 251.81 108.8519) (end 253.01 107.6519) (width 0.4) (layer "B.Cu") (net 11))
 (segment (start 253.01 106.4) (end 253.01 105.1481) (width 0.4) (layer "B.Cu") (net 11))
 (segment (start 251.81 110) (end 251.81 108.8519) (width 0.4) (layer "B.Cu") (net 11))
 (segment (start 253.01 105.1481) (end 251.81 103.9481) (width 0.4) (layer "B.Cu") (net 11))
 (segment (start 270.79 104.25) (end 270.79 106.4) (width 0.4) (layer "B.Cu") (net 10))
 (segment (start 268.089999 101.55) (end 270.79 104.25) (width 0.4) (layer "B.Cu") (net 10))
 (segment (start 270.79 107.6519) (end 270.4381 107.6519) (width 0.4) (layer "B.Cu") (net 10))
 (segment (start 270.79 106.4) (end 270.79 107.6519) (width 0.4) (layer "B.Cu") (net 10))
 (segment (start 270.4381 107.6519) (end 268.089999 110) (width 0.4) (layer "B.Cu") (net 10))
 (segment (start 181.78 109.56) (end 207.09 109.56) (width 0.4) (layer "F.Cu") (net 4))
 (segment (start 207.09 109.56) (end 210.35 106.3) (width 0.4) (layer "F.Cu") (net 4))
 (segment (start 212.53 104.48) (end 214.35 106.3) (width 0.4) (layer "F.Cu") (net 5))
 (segment (start 181.78 104.48) (end 212.53 104.48) (width 0.4) (layer "F.Cu") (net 5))
 (segment (start 184.5838 101.8423) (end 184.4861 101.94) (width 0.4) (layer "F.Cu") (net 6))
 (segment (start 216.35 106.3) (end 211.9392 101.8892) (width 0.4) (layer "F.Cu") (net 6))
 (segment (start 211.9392 101.8892) (end 211.9392 100.9304) (width 0.4) (layer "F.Cu") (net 6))
 (segment (start 184.4861 101.94) (end 181.78 101.94) (width 0.4) (layer "F.Cu") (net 6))
 (via (at 184.5838 101.8423) (size 0.8) (drill 0.4) (layers "F.Cu" "B.Cu") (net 6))
 (via (at 211.9392 100.9304) (size 0.8) (drill 0.4) (layers "F.Cu" "B.Cu") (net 6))
 (segment (start 185.4957 100.9304) (end 184.5838 101.8423) (width 0.4) (layer "B.Cu") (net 6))
 (segment (start 211.9392 100.9304) (end 185.4957 100.9304) (width 0.4) (layer "B.Cu") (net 6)))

